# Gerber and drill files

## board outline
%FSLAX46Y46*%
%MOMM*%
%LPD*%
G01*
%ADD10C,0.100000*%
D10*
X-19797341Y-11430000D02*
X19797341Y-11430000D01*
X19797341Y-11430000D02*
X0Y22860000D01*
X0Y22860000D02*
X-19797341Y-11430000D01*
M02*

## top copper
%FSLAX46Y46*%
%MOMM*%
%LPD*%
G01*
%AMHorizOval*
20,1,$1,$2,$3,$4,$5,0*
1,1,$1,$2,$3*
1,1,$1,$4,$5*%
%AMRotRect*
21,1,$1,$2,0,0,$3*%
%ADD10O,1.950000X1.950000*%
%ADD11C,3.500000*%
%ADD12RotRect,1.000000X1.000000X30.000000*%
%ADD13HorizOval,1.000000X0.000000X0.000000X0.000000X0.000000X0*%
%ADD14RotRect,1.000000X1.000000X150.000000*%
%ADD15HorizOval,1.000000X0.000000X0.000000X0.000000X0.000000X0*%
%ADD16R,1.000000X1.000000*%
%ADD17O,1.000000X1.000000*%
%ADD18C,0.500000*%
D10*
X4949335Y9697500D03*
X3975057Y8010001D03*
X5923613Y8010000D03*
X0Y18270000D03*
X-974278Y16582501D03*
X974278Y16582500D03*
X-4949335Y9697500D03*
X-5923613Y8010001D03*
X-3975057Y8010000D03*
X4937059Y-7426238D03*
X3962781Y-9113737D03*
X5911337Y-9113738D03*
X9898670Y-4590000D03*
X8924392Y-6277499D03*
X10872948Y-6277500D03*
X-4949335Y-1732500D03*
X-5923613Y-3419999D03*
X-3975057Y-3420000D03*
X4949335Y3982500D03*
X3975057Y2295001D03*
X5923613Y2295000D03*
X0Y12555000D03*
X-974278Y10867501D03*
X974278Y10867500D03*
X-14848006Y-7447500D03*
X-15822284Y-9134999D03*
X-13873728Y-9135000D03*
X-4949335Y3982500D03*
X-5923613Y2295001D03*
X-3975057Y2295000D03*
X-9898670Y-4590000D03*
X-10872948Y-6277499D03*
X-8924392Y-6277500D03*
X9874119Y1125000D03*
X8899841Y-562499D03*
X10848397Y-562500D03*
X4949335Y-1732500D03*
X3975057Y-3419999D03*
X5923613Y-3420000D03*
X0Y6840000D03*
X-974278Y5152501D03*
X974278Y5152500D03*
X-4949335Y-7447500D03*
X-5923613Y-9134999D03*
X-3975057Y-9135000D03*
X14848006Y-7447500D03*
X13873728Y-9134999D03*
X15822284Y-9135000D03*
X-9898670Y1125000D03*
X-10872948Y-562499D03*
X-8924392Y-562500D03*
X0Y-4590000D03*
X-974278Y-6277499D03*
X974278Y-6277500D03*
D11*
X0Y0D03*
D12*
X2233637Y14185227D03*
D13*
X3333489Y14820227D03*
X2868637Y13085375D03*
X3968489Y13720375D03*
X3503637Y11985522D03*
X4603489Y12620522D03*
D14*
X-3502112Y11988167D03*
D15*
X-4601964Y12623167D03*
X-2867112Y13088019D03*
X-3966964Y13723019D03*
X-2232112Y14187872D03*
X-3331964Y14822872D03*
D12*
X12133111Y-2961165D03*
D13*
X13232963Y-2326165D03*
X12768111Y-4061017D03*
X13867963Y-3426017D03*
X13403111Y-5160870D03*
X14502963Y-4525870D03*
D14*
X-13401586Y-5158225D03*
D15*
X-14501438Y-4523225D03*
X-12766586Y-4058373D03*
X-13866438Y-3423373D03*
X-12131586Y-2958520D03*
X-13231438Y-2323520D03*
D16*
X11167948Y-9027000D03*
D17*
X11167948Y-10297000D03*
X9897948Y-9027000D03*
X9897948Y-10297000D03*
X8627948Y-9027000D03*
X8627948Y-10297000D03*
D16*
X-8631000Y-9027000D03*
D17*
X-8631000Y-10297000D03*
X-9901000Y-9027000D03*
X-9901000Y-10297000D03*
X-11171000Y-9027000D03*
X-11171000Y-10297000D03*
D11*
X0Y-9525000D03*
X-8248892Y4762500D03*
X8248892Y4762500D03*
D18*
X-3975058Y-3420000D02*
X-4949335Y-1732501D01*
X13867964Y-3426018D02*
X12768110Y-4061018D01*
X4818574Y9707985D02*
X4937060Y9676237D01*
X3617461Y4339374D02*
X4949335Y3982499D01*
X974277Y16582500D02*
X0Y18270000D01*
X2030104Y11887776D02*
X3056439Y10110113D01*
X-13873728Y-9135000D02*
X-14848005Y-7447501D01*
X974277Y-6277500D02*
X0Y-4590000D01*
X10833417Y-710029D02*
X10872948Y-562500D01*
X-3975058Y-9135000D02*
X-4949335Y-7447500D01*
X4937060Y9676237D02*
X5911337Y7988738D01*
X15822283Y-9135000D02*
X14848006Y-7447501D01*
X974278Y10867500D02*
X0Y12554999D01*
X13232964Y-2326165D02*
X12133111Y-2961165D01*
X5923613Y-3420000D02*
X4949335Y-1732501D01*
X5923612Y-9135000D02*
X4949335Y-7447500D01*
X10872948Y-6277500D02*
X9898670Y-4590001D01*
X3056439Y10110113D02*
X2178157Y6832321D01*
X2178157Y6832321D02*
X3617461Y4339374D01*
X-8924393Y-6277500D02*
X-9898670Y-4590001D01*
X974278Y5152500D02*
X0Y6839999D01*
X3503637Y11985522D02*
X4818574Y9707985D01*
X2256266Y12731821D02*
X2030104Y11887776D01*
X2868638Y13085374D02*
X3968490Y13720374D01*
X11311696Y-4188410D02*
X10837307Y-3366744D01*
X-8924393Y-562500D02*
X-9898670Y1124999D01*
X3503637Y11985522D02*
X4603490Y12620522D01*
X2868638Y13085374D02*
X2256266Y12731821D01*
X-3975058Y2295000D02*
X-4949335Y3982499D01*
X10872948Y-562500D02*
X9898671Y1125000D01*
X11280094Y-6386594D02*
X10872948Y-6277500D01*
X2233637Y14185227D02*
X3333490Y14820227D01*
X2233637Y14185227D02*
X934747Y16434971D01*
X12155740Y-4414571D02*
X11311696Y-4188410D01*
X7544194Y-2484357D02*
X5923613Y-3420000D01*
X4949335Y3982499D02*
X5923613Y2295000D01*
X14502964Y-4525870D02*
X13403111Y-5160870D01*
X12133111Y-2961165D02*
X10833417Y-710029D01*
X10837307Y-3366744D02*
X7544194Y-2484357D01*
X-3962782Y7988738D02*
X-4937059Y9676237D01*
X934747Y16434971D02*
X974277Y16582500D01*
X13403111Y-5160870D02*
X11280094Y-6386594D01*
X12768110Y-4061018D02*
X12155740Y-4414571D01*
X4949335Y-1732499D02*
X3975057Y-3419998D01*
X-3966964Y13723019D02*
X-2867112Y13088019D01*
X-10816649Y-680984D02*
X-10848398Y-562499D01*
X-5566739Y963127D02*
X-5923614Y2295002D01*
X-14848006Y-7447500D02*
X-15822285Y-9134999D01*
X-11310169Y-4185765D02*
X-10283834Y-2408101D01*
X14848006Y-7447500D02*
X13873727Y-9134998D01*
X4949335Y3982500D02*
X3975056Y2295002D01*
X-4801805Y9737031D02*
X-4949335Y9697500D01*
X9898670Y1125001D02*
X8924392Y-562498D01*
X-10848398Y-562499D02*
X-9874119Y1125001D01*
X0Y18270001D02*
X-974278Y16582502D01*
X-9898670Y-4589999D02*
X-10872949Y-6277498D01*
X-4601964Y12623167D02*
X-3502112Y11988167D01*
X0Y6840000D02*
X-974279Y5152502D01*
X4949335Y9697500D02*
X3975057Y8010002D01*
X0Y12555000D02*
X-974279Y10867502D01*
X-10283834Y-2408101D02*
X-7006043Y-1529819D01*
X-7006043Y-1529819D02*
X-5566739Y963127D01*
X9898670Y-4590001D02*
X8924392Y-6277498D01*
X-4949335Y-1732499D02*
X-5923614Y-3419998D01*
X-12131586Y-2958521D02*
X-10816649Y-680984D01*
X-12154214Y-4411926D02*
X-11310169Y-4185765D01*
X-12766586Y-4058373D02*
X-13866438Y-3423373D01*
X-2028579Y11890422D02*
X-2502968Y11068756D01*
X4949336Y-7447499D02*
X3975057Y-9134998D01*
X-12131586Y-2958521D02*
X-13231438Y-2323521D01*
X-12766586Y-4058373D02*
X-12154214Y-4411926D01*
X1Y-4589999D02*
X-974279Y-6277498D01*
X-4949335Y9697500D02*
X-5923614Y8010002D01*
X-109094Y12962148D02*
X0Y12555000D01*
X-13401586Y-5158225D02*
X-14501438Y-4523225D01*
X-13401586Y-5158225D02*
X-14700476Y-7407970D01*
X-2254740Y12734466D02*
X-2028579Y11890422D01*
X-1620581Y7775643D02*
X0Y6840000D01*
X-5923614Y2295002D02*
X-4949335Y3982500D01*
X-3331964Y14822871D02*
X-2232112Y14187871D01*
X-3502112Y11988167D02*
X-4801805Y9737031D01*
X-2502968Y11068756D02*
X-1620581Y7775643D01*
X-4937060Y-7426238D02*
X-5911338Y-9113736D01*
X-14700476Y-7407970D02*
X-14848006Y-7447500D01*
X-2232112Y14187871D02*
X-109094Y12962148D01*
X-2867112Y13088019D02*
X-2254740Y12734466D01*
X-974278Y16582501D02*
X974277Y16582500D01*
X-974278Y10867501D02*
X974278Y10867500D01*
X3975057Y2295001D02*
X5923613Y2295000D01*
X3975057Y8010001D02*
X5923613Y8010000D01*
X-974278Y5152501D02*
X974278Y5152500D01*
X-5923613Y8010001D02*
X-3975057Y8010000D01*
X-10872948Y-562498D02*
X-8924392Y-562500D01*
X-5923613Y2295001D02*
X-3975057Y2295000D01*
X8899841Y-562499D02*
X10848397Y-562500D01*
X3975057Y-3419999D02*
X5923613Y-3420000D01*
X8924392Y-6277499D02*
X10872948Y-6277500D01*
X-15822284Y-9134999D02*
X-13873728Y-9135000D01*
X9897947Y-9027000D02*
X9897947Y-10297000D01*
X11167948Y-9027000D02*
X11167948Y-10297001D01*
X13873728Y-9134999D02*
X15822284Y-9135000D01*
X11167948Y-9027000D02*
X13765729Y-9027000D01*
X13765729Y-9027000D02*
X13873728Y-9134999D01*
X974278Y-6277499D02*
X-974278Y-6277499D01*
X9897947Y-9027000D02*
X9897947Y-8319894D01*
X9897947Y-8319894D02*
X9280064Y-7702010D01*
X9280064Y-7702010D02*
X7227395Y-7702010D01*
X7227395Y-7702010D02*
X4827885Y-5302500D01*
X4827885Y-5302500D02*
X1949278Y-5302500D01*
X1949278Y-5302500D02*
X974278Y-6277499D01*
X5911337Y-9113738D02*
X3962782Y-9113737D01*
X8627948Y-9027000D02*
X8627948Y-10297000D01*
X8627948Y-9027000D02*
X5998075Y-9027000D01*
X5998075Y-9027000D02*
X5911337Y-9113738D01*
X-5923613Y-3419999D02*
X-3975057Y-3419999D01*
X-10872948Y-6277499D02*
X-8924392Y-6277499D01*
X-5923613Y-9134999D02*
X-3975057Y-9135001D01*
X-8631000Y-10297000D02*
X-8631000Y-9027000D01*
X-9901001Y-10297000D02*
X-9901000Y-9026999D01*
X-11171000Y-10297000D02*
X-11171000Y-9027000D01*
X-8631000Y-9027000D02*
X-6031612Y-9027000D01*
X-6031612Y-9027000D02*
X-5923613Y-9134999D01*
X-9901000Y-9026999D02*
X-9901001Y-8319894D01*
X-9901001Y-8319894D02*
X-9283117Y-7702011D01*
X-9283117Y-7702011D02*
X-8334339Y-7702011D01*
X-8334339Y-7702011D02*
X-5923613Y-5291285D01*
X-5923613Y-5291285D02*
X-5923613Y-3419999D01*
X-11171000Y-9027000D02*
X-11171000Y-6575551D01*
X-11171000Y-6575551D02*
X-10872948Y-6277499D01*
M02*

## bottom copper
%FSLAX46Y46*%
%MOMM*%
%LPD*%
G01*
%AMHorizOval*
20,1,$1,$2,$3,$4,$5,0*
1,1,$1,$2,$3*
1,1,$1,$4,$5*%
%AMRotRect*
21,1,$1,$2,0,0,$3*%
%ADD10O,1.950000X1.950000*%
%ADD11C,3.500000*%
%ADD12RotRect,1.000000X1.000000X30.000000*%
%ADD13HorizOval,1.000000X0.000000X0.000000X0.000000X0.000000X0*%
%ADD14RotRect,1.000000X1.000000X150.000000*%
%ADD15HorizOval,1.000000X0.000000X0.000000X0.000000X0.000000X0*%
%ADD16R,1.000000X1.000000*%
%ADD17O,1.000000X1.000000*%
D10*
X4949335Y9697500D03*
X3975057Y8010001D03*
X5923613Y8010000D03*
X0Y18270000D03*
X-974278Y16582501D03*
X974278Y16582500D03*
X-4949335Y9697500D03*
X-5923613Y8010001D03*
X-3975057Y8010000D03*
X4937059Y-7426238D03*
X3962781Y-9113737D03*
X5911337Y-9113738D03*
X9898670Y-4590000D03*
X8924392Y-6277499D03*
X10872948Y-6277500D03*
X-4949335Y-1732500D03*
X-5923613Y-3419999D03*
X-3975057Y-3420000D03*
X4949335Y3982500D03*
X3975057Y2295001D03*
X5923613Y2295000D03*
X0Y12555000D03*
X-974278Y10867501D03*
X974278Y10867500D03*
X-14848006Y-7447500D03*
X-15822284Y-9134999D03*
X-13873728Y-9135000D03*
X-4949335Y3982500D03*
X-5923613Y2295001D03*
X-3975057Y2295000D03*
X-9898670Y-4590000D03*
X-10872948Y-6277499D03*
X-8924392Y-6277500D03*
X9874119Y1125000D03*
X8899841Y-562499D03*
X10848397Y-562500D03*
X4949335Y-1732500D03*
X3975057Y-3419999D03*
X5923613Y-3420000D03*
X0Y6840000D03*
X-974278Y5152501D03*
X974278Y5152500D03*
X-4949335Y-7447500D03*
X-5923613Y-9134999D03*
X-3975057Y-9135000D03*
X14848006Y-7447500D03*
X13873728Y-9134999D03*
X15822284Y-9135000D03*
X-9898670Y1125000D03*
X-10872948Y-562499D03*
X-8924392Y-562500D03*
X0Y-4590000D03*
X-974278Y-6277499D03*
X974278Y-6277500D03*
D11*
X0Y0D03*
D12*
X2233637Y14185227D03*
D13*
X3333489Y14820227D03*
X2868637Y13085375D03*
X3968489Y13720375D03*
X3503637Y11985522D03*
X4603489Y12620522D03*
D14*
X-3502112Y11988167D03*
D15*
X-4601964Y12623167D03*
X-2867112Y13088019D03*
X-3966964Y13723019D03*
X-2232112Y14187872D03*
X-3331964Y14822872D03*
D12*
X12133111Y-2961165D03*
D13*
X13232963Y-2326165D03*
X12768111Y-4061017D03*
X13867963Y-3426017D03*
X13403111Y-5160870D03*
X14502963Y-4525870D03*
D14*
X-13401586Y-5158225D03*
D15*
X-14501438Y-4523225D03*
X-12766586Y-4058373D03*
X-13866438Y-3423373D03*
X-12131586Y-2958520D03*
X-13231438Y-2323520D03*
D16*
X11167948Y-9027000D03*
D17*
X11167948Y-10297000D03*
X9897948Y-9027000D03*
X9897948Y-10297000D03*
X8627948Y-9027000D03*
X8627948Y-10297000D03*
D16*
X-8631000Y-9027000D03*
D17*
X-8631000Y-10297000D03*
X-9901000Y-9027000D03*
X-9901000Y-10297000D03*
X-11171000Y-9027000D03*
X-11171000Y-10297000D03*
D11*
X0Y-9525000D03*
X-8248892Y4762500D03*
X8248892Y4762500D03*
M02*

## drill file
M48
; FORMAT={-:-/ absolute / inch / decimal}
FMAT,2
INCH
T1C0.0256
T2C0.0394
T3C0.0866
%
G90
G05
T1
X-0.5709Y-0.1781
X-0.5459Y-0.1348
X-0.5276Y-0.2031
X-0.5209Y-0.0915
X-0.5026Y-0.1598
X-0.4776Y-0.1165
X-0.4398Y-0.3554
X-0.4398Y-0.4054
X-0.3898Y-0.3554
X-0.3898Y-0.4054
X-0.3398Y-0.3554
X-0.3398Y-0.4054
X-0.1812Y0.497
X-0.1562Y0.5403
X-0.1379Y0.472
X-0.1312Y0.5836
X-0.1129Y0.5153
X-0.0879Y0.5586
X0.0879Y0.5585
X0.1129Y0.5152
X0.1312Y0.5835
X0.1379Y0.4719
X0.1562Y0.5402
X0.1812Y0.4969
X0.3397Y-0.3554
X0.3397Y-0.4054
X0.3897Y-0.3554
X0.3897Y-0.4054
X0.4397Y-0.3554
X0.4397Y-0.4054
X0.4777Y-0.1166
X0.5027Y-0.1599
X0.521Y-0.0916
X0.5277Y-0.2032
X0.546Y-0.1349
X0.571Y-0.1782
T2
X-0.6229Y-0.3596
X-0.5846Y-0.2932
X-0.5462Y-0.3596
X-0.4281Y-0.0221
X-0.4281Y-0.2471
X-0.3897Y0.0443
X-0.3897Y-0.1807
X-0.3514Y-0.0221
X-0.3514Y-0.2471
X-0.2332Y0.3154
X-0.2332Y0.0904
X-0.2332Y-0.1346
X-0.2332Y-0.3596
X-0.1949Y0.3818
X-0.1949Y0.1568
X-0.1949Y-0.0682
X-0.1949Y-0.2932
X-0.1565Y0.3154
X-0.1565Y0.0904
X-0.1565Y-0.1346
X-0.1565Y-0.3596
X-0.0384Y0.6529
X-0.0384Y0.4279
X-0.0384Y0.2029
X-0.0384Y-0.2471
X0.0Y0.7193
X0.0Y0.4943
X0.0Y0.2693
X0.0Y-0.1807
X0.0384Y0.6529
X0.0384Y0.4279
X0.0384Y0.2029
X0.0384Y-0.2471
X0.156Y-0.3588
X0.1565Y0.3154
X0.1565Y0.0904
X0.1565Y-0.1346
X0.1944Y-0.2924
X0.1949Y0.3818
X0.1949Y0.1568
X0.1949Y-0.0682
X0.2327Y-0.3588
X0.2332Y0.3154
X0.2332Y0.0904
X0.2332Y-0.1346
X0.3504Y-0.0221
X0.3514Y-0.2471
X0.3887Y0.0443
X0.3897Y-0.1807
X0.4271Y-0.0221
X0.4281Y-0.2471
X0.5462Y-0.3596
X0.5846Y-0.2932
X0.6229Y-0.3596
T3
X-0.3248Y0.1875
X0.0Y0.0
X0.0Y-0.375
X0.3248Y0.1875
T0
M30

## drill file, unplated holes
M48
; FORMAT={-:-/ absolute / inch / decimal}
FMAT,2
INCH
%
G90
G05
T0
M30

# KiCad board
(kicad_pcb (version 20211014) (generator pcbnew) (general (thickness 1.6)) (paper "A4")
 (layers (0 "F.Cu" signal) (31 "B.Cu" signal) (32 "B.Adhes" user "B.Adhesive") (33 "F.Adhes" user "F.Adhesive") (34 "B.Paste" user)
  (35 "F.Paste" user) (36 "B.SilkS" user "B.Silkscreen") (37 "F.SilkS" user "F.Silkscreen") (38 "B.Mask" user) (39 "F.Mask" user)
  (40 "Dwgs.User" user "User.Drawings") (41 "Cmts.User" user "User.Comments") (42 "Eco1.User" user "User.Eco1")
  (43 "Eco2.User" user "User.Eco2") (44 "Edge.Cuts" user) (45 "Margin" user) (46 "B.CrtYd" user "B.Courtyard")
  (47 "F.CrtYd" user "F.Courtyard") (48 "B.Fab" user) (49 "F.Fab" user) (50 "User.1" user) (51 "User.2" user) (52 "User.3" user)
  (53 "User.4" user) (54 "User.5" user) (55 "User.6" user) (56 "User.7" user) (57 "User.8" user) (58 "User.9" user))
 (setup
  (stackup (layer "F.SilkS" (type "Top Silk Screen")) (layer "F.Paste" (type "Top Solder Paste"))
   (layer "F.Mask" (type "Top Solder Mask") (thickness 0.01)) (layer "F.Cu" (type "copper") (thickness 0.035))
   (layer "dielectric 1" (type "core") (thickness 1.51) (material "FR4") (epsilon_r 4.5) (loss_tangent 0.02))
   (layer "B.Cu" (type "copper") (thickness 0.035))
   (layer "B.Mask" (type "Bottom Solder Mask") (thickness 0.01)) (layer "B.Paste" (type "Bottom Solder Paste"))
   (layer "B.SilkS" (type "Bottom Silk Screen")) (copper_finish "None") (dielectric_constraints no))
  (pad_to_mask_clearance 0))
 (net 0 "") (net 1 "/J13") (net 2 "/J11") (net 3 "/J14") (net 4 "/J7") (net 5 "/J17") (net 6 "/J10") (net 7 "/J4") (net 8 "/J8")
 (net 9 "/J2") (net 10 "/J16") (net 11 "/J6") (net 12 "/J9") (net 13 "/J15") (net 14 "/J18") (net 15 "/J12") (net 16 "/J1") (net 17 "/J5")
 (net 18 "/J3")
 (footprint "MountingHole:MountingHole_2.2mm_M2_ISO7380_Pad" (layer "F.Cu") (at 0 9.525)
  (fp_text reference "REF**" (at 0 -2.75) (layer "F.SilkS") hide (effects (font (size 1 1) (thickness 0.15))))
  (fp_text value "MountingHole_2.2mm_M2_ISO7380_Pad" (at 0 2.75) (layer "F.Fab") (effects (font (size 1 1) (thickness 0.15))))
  (pad "1" thru_hole circle (at 0 0) (size 3.5 3.5) (drill 2.2) (layers *.Cu *.Mask)))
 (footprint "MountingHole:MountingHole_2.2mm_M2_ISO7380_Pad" (layer "F.Cu") (at 0 0)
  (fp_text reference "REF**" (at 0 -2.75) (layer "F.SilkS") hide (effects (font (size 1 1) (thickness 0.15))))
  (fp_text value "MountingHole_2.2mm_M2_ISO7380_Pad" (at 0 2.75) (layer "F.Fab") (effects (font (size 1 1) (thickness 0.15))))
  (pad "1" thru_hole circle (at 0 0) (size 3.5 3.5) (drill 2.2) (layers *.Cu *.Mask)))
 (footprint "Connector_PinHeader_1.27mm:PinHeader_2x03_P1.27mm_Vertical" (layer "F.Cu") (at 11.167948 9.027 -90)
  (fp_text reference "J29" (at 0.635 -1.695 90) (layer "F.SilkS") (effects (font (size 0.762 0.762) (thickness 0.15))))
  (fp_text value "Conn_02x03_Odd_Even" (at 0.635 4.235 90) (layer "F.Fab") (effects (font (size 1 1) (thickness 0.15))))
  (pad "1" thru_hole rect (at 0 0 270) (size 1 1) (drill 0.65) (layers *.Cu *.Mask) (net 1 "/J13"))
  (pad "2" thru_hole oval (at 1.27 0 270) (size 1 1) (drill 0.65) (layers *.Cu *.Mask) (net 1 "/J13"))
  (pad "3" thru_hole oval (at 0 1.27 270) (size 1 1) (drill 0.65) (layers *.Cu *.Mask) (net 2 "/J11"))
  (pad "4" thru_hole oval (at 1.27 1.27 270) (size 1 1) (drill 0.65) (layers *.Cu *.Mask) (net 2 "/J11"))
  (pad "5" thru_hole oval (at 0 2.54 270) (size 1 1) (drill 0.65) (layers *.Cu *.Mask) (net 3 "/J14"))
  (pad "6" thru_hole oval (at 1.27 2.54 270) (size 1 1) (drill 0.65) (layers *.Cu *.Mask) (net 3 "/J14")))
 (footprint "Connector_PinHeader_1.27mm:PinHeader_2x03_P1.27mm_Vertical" (layer "F.Cu") (at 12.133111 2.961165 30)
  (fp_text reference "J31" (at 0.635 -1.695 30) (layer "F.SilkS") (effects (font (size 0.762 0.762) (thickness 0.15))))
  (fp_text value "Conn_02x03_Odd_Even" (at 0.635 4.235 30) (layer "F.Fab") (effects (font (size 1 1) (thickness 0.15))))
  (pad "1" thru_hole rect (at 0 0 30) (size 1 1) (drill 0.65) (layers *.Cu *.Mask) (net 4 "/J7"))
  (pad "2" thru_hole oval (at 1.27 0 30) (size 1 1) (drill 0.65) (layers *.Cu *.Mask) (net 4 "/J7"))
  (pad "3" thru_hole oval (at 0 1.27 30) (size 1 1) (drill 0.65) (layers *.Cu *.Mask) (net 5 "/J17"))
  (pad "4" thru_hole oval (at 1.27 1.27 30) (size 1 1) (drill 0.65) (layers *.Cu *.Mask) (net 5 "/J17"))
  (pad "5" thru_hole oval (at 0 2.54 30) (size 1 1) (drill 0.65) (layers *.Cu *.Mask) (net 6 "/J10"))
  (pad "6" thru_hole oval (at 1.27 2.54 30) (size 1 1) (drill 0.65) (layers *.Cu *.Mask) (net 6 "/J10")))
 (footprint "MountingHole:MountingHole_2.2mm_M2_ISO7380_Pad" (layer "F.Cu") (at -8.248892 -4.7625)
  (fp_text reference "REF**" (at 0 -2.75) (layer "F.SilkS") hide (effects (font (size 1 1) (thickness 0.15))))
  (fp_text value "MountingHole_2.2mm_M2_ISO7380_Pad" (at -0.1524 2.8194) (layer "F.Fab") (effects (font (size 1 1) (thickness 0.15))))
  (pad "1" thru_hole circle (at 0 0) (size 3.5 3.5) (drill 2.2) (layers *.Cu *.Mask)))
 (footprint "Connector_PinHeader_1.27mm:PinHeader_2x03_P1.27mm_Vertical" (layer "F.Cu") (at -3.502112 -11.988167 150)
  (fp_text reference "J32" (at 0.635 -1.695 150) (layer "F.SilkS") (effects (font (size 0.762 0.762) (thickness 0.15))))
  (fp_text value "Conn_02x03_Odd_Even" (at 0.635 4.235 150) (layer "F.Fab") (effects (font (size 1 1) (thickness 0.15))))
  (pad "1" thru_hole rect (at 0 0 150) (size 1 1) (drill 0.65) (layers *.Cu *.Mask) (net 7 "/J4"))
  (pad "2" thru_hole oval (at 1.27 0 150) (size 1 1) (drill 0.65) (layers *.Cu *.Mask) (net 7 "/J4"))
  (pad "3" thru_hole oval (at 0 1.27 150) (size 1 1) (drill 0.65) (layers *.Cu *.Mask) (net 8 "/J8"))
  (pad "4" thru_hole oval (at 1.27 1.27 150) (size 1 1) (drill 0.65) (layers *.Cu *.Mask) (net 8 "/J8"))
  (pad "5" thru_hole oval (at 0 2.54 150) (size 1 1) (drill 0.65) (layers *.Cu *.Mask) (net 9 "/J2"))
  (pad "6" thru_hole oval (at 1.27 2.54 150) (size 1 1) (drill 0.65) (layers *.Cu *.Mask) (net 9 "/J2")))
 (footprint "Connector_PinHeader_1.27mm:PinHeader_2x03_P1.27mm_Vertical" (layer "F.Cu") (at -13.401586 5.158225 150)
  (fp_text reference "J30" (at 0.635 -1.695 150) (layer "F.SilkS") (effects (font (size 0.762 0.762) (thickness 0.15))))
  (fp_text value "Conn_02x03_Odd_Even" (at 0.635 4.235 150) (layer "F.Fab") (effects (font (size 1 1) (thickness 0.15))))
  (pad "1" thru_hole rect (at 0 0 150) (size 1 1) (drill 0.65) (layers *.Cu *.Mask) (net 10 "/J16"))
  (pad "2" thru_hole oval (at 1.27 0 150) (size 1 1) (drill 0.65) (layers *.Cu *.Mask) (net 10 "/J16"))
  (pad "3" thru_hole oval (at 0 1.27 150) (size 1 1) (drill 0.65) (layers *.Cu *.Mask) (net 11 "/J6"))
  (pad "4" thru_hole oval (at 1.27 1.27 150) (size 1 1) (drill 0.65) (layers *.Cu *.Mask) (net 11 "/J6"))
  (pad "5" thru_hole oval (at 0 2.54 150) (size 1 1) (drill 0.65) (layers *.Cu *.Mask) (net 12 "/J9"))
  (pad "6" thru_hole oval (at 1.27 2.54 150) (size 1 1) (drill 0.65) (layers *.Cu *.Mask) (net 12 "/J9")))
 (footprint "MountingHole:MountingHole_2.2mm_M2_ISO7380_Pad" (layer "F.Cu") (at 8.248892 -4.7625)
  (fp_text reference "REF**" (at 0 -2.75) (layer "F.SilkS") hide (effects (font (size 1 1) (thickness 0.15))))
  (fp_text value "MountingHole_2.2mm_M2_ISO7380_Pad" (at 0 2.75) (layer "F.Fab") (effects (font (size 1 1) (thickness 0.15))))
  (pad "1" thru_hole circle (at 0 0) (size 3.5 3.5) (drill 2.2) (layers *.Cu *.Mask)))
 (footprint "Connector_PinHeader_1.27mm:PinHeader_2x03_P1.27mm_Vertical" (layer "F.Cu") (at -8.631 9.027 -90)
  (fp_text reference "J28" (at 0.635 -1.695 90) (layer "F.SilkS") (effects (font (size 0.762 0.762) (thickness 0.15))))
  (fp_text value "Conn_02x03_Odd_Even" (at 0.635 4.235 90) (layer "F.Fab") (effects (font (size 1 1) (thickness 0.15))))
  (pad "1" thru_hole rect (at 0 0 270) (size 1 1) (drill 0.65) (layers *.Cu *.Mask) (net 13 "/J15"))
  (pad "2" thru_hole oval (at 1.27 0 270) (size 1 1) (drill 0.65) (layers *.Cu *.Mask) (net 13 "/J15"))
  (pad "3" thru_hole oval (at 0 1.27 270) (size 1 1) (drill 0.65) (layers *.Cu *.Mask) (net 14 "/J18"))
  (pad "4" thru_hole oval (at 1.27 1.27 270) (size 1 1) (drill 0.65) (layers *.Cu *.Mask) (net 14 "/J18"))
  (pad "5" thru_hole oval (at 0 2.54 270) (size 1 1) (drill 0.65) (layers *.Cu *.Mask) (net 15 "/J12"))
  (pad "6" thru_hole oval (at 1.27 2.54 270) (size 1 1) (drill 0.65) (layers *.Cu *.Mask) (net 15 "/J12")))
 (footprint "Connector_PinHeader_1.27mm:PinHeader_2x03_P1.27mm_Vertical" (layer "F.Cu") (at 2.233637 -14.185227 30)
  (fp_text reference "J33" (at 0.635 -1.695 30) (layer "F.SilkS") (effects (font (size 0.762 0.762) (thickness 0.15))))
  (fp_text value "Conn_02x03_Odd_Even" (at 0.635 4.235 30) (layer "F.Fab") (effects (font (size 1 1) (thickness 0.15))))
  (pad "1" thru_hole rect (at 0 0 30) (size 1 1) (drill 0.65) (layers *.Cu *.Mask) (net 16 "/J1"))
  (pad "2" thru_hole oval (at 1.27 0 30) (size 1 1) (drill 0.65) (layers *.Cu *.Mask) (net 16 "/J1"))
  (pad "3" thru_hole oval (at 0 1.27 30) (size 1 1) (drill 0.65) (layers *.Cu *.Mask) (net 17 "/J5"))
  (pad "4" thru_hole oval (at 1.27 1.27 30) (size 1 1) (drill 0.65) (layers *.Cu *.Mask) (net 17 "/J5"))
  (pad "5" thru_hole oval (at 0 2.54 30) (size 1 1) (drill 0.65) (layers *.Cu *.Mask) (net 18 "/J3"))
  (pad "6" thru_hole oval (at 1.27 2.54 30) (size 1 1) (drill 0.65) (layers *.Cu *.Mask) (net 18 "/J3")))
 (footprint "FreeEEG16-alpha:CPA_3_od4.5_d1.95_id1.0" (layer "B.Cu") (at 0 -17.145 180)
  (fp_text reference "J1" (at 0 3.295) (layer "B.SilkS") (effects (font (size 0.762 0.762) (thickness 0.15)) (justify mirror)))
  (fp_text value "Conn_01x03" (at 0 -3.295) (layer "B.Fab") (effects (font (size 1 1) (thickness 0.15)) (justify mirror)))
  (pad "1" thru_hole oval (at 0 1.125 180) (size 1.95 1.95) (drill 1) (layers *.Cu *.Mask) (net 16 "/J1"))
  (pad "2" thru_hole oval (at 0.974278 -0.562499 180) (size 1.95 1.95) (drill 1) (layers *.Cu *.Mask) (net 16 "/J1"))
  (pad "3" thru_hole oval (at -0.974278 -0.5625 180) (size 1.95 1.95) (drill 1) (layers *.Cu *.Mask) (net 16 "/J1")))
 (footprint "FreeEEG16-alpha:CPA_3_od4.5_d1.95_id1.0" (layer "B.Cu") (at -4.949335 -8.5725 180)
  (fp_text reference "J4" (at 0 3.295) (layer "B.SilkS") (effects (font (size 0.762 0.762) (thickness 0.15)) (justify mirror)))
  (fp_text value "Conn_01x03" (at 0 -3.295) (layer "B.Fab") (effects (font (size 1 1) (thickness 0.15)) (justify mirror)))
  (pad "1" thru_hole oval (at 0 1.125 180) (size 1.95 1.95) (drill 1) (layers *.Cu *.Mask) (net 7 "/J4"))
  (pad "2" thru_hole oval (at 0.974278 -0.562499 180) (size 1.95 1.95) (drill 1) (layers *.Cu *.Mask) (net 7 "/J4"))
  (pad "3" thru_hole oval (at -0.974278 -0.5625 180) (size 1.95 1.95) (drill 1) (layers *.Cu *.Mask) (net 7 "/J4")))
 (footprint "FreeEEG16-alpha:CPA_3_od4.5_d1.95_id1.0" (layer "B.Cu") (at 4.937059 8.551238 180)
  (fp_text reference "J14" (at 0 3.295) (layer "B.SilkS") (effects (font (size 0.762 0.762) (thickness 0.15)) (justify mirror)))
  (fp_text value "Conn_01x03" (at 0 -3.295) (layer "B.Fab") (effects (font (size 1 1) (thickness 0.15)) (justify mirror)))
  (pad "1" thru_hole oval (at 0 1.125 180) (size 1.95 1.95) (drill 1) (layers *.Cu *.Mask) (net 3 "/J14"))
  (pad "2" thru_hole oval (at 0.974278 -0.562499 180) (size 1.95 1.95) (drill 1) (layers *.Cu *.Mask) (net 3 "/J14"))
  (pad "3" thru_hole oval (at -0.974278 -0.5625 180) (size 1.95 1.95) (drill 1) (layers *.Cu *.Mask) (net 3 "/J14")))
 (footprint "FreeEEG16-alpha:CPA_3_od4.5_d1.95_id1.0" (layer "B.Cu") (at 4.949335 -8.5725 180)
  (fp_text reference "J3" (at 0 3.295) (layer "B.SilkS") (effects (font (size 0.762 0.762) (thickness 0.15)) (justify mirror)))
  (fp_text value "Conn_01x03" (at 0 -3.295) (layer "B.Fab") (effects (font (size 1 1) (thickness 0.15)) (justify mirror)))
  (pad "1" thru_hole oval (at 0 1.125 180) (size 1.95 1.95) (drill 1) (layers *.Cu *.Mask) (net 18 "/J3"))
  (pad "2" thru_hole oval (at 0.974278 -0.562499 180) (size 1.95 1.95) (drill 1) (layers *.Cu *.Mask) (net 18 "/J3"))
  (pad "3" thru_hole oval (at -0.974278 -0.5625 180) (size 1.95 1.95) (drill 1) (layers *.Cu *.Mask) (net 18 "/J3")))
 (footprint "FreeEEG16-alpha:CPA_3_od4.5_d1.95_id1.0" (layer "B.Cu") (at 9.89867 5.715 180)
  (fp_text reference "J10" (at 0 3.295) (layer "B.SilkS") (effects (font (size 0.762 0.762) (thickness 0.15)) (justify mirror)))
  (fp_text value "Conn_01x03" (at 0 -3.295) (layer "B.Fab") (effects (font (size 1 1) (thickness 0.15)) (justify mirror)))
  (pad "1" thru_hole oval (at 0 1.125 180) (size 1.95 1.95) (drill 1) (layers *.Cu *.Mask) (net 6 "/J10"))
  (pad "2" thru_hole oval (at 0.974278 -0.562499 180) (size 1.95 1.95) (drill 1) (layers *.Cu *.Mask) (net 6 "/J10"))
  (pad "3" thru_hole oval (at -0.974278 -0.5625 180) (size 1.95 1.95) (drill 1) (layers *.Cu *.Mask) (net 6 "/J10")))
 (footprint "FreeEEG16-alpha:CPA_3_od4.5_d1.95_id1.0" (layer "B.Cu") (at -4.949335 2.8575 180)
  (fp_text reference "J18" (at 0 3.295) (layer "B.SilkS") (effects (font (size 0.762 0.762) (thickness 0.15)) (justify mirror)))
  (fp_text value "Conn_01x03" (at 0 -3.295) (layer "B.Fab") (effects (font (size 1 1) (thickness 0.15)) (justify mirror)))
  (pad "1" thru_hole oval (at 0 1.125 180) (size 1.95 1.95) (drill 1) (layers *.Cu *.Mask) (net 14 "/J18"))
  (pad "2" thru_hole oval (at 0.974278 -0.562499 180) (size 1.95 1.95) (drill 1) (layers *.Cu *.Mask) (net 14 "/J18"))
  (pad "3" thru_hole oval (at -0.974278 -0.5625 180) (size 1.95 1.95) (drill 1) (layers *.Cu *.Mask) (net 14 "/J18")))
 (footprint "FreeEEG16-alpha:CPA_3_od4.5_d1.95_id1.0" (layer "B.Cu") (at 4.949335 -2.8575 180)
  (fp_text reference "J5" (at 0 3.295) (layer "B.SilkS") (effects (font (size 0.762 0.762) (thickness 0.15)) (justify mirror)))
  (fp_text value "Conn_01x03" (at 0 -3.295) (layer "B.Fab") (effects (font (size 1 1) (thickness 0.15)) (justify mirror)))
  (pad "1" thru_hole oval (at 0 1.125 180) (size 1.95 1.95) (drill 1) (layers *.Cu *.Mask) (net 17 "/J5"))
  (pad "2" thru_hole oval (at 0.974278 -0.562499 180) (size 1.95 1.95) (drill 1) (layers *.Cu *.Mask) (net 17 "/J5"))
  (pad "3" thru_hole oval (at -0.974278 -0.5625 180) (size 1.95 1.95) (drill 1) (layers *.Cu *.Mask) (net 17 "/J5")))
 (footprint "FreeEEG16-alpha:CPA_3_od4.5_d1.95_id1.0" (layer "B.Cu") (at 0 -11.43 180)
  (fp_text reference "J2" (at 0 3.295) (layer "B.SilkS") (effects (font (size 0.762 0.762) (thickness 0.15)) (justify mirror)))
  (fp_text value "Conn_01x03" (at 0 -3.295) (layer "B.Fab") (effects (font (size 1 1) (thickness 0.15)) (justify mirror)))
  (pad "1" thru_hole oval (at 0 1.125 180) (size 1.95 1.95) (drill 1) (layers *.Cu *.Mask) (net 9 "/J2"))
  (pad "2" thru_hole oval (at 0.974278 -0.562499 180) (size 1.95 1.95) (drill 1) (layers *.Cu *.Mask) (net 9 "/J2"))
  (pad "3" thru_hole oval (at -0.974278 -0.5625 180) (size 1.95 1.95) (drill 1) (layers *.Cu *.Mask) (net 9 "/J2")))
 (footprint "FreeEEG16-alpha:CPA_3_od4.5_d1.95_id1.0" (layer "B.Cu") (at -14.848006 8.5725 180)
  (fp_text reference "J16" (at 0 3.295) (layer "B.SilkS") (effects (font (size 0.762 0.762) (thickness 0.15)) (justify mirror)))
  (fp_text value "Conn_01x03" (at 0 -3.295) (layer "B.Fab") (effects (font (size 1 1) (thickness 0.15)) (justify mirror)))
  (pad "1" thru_hole oval (at 0 1.125 180) (size 1.95 1.95) (drill 1) (layers *.Cu *.Mask) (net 10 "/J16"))
  (pad "2" thru_hole oval (at 0.974278 -0.562499 180) (size 1.95 1.95) (drill 1) (layers *.Cu *.Mask) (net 10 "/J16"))
  (pad "3" thru_hole oval (at -0.974278 -0.5625 180) (size 1.95 1.95) (drill 1) (layers *.Cu *.Mask) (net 10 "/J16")))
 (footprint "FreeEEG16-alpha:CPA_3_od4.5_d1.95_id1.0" (layer "B.Cu") (at -4.949335 -2.8575 180)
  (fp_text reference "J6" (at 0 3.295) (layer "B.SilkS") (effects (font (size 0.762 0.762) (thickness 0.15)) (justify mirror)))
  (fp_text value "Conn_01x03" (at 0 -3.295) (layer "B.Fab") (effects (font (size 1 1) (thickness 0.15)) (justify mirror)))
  (pad "1" thru_hole oval (at 0 1.125 180) (size 1.95 1.95) (drill 1) (layers *.Cu *.Mask) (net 11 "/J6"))
  (pad "2" thru_hole oval (at 0.974278 -0.562499 180) (size 1.95 1.95) (drill 1) (layers *.Cu *.Mask) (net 11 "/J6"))
  (pad "3" thru_hole oval (at -0.974278 -0.5625 180) (size 1.95 1.95) (drill 1) (layers *.Cu *.Mask) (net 11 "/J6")))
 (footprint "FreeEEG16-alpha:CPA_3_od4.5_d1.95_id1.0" (layer "B.Cu") (at -9.89867 5.715 180)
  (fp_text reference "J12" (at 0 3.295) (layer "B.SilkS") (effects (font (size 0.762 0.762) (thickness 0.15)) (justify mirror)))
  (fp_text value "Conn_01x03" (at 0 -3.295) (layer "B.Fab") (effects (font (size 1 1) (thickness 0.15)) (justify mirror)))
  (pad "1" thru_hole oval (at 0 1.125 180) (size 1.95 1.95) (drill 1) (layers *.Cu *.Mask) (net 15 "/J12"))
  (pad "2" thru_hole oval (at 0.974278 -0.562499 180) (size 1.95 1.95) (drill 1) (layers *.Cu *.Mask) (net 15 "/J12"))
  (pad "3" thru_hole oval (at -0.974278 -0.5625 180) (size 1.95 1.95) (drill 1) (layers *.Cu *.Mask) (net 15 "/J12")))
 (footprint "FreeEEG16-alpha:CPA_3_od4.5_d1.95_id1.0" (layer "B.Cu") (at 9.874119 0 180)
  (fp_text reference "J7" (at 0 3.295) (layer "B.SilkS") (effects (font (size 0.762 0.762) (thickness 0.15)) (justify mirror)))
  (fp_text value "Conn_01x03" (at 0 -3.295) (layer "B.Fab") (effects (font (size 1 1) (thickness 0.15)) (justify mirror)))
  (pad "1" thru_hole oval (at 0 1.125 180) (size 1.95 1.95) (drill 1) (layers *.Cu *.Mask) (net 4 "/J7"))
  (pad "2" thru_hole oval (at 0.974278 -0.562499 180) (size 1.95 1.95) (drill 1) (layers *.Cu *.Mask) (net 4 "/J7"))
  (pad "3" thru_hole oval (at -0.974278 -0.5625 180) (size 1.95 1.95) (drill 1) (layers *.Cu *.Mask) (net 4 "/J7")))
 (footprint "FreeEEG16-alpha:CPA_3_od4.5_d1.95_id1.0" (layer "B.Cu") (at 4.949335 2.8575 180)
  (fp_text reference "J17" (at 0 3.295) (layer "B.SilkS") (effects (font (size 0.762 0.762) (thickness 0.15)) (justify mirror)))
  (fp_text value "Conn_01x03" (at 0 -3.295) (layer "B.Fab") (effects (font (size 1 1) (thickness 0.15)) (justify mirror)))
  (pad "1" thru_hole oval (at 0 1.125 180) (size 1.95 1.95) (drill 1) (layers *.Cu *.Mask) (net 5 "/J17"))
  (pad "2" thru_hole oval (at 0.974278 -0.562499 180) (size 1.95 1.95) (drill 1) (layers *.Cu *.Mask) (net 5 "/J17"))
  (pad "3" thru_hole oval (at -0.974278 -0.5625 180) (size 1.95 1.95) (drill 1) (layers *.Cu *.Mask) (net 5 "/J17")))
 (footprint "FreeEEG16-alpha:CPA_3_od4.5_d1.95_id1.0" (layer "B.Cu") (at 0 -5.715 180)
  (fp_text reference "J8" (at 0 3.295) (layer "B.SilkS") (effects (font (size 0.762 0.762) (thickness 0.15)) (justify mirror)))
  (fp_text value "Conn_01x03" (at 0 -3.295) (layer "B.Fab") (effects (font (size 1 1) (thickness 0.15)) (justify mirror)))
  (pad "1" thru_hole oval (at 0 1.125 180) (size 1.95 1.95) (drill 1) (layers *.Cu *.Mask) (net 8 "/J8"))
  (pad "2" thru_hole oval (at 0.974278 -0.562499 180) (size 1.95 1.95) (drill 1) (layers *.Cu *.Mask) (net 8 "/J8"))
  (pad "3" thru_hole oval (at -0.974278 -0.5625 180) (size 1.95 1.95) (drill 1) (layers *.Cu *.Mask) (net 8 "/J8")))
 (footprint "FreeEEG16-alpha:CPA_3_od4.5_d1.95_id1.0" (layer "B.Cu") (at -4.949335 8.5725 180)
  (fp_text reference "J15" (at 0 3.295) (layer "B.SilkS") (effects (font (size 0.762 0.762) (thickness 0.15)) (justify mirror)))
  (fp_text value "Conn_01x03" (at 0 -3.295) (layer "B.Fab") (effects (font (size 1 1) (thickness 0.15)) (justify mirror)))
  (pad "1" thru_hole oval (at 0 1.125 180) (size 1.95 1.95) (drill 1) (layers *.Cu *.Mask) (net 13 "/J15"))
  (pad "2" thru_hole oval (at 0.974278 -0.562499 180) (size 1.95 1.95) (drill 1) (layers *.Cu *.Mask) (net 13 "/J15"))
  (pad "3" thru_hole oval (at -0.974278 -0.5625 180) (size 1.95 1.95) (drill 1) (layers *.Cu *.Mask) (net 13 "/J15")))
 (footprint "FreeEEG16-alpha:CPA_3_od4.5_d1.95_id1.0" (layer "B.Cu") (at 14.848006 8.5725 180)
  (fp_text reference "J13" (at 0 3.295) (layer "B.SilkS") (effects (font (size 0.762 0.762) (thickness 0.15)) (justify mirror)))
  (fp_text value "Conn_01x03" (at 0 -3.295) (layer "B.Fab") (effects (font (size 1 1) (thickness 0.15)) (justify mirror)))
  (pad "1" thru_hole oval (at 0 1.125 180) (size 1.95 1.95) (drill 1) (layers *.Cu *.Mask) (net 1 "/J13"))
  (pad "2" thru_hole oval (at 0.974278 -0.562499 180) (size 1.95 1.95) (drill 1) (layers *.Cu *.Mask) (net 1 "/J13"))
  (pad "3" thru_hole oval (at -0.974278 -0.5625 180) (size 1.95 1.95) (drill 1) (layers *.Cu *.Mask) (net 1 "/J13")))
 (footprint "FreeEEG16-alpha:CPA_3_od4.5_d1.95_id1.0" (layer "B.Cu") (at -9.89867 0 180)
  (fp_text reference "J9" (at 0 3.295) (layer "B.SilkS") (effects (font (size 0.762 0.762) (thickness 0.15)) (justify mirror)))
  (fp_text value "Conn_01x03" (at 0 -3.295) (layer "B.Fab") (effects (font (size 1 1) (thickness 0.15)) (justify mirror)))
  (pad "1" thru_hole oval (at 0 1.125 180) (size 1.95 1.95) (drill 1) (layers *.Cu *.Mask) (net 12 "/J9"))
  (pad "2" thru_hole oval (at 0.974278 -0.562499 180) (size 1.95 1.95) (drill 1) (layers *.Cu *.Mask) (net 12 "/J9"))
  (pad "3" thru_hole oval (at -0.974278 -0.5625 180) (size 1.95 1.95) (drill 1) (layers *.Cu *.Mask) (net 12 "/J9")))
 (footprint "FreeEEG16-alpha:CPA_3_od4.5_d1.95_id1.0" (layer "B.Cu") (at 0 5.715 180)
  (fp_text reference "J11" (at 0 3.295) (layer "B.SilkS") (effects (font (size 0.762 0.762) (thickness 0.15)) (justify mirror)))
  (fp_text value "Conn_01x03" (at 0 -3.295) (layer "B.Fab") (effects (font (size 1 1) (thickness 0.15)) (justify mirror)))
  (pad "1" thru_hole oval (at 0 1.125 180) (size 1.95 1.95) (drill 1) (layers *.Cu *.Mask) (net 2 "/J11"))
  (pad "2" thru_hole oval (at 0.974278 -0.562499 180) (size 1.95 1.95) (drill 1) (layers *.Cu *.Mask) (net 2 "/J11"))
  (pad "3" thru_hole oval (at -0.974278 -0.5625 180) (size 1.95 1.95) (drill 1) (layers *.Cu *.Mask) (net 2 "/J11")))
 (gr_line (start -19.797341 11.43) (end 19.797341 11.43) (layer "Edge.Cuts") (width 0.1))
 (gr_line (start 19.797341 11.43) (end 0 -22.86) (layer "Edge.Cuts") (width 0.1))
 (gr_line (start 0 -22.86) (end -19.797341 11.43) (layer "Edge.Cuts") (width 0.1))
 (segment (start 0 -18.270001) (end -0.974278 -16.582502) (width 0.5) (layer "F.Cu") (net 16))
 (segment (start 0.934747 -16.434971) (end 0.974277 -16.5825) (width 0.5) (layer "F.Cu") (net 16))
 (segment (start 0.974277 -16.5825) (end 0 -18.27) (width 0.5) (layer "F.Cu") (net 16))
 (segment (start -0.974278 -16.582501) (end 0.974277 -16.5825) (width 0.5) (layer "F.Cu") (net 16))
 (segment (start 2.233637 -14.185227) (end 0.934747 -16.434971) (width 0.5) (layer "F.Cu") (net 16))
 (segment (start 2.233637 -14.185227) (end 3.33349 -14.820227) (width 0.5) (layer "F.Cu") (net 16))
 (segment (start -2.232112 -14.187871) (end -0.109094 -12.962148) (width 0.5) (layer "F.Cu") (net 9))
 (segment (start 0 -12.555) (end -0.974279 -10.867502) (width 0.5) (layer "F.Cu") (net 9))
 (segment (start -0.974278 -10.867501) (end 0.974278 -10.8675) (width 0.5) (layer "F.Cu") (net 9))
 (segment (start -3.331964 -14.822871) (end -2.232112 -14.187871) (width 0.5) (layer "F.Cu") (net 9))
 (segment (start -0.109094 -12.962148) (end 0 -12.555) (width 0.5) (layer "F.Cu") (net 9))
 (segment (start 0.974278 -10.8675) (end 0 -12.554999) (width 0.5) (layer "F.Cu") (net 9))
 (segment (start 4.818574 -9.707985) (end 4.93706 -9.676237) (width 0.5) (layer "F.Cu") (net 18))
 (segment (start 3.503637 -11.985522) (end 4.818574 -9.707985) (width 0.5) (layer "F.Cu") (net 18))
 (segment (start 3.975057 -8.010001) (end 5.923613 -8.01) (width 0.5) (layer "F.Cu") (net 18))
 (segment (start 4.93706 -9.676237) (end 5.911337 -7.988738) (width 0.5) (layer "F.Cu") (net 18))
 (segment (start 4.949335 -9.6975) (end 3.975057 -8.010002) (width 0.5) (layer "F.Cu") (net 18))
 (segment (start 3.503637 -11.985522) (end 4.60349 -12.620522) (width 0.5) (layer "F.Cu") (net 18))
 (segment (start -4.601964 -12.623167) (end -3.502112 -11.988167) (width 0.5) (layer "F.Cu") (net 7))
 (segment (start -3.962782 -7.988738) (end -4.937059 -9.676237) (width 0.5) (layer "F.Cu") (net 7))
 (segment (start -4.801805 -9.737031) (end -4.949335 -9.6975) (width 0.5) (layer "F.Cu") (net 7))
 (segment (start -3.502112 -11.988167) (end -4.801805 -9.737031) (width 0.5) (layer "F.Cu") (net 7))
 (segment (start -5.923613 -8.010001) (end -3.975057 -8.01) (width 0.5) (layer "F.Cu") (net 7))
 (segment (start -4.949335 -9.6975) (end -5.923614 -8.010002) (width 0.5) (layer "F.Cu") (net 7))
 (segment (start 4.949335 -3.9825) (end 3.975056 -2.295002) (width 0.5) (layer "F.Cu") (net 17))
 (segment (start 2.178157 -6.832321) (end 3.617461 -4.339374) (width 0.5) (layer "F.Cu") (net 17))
 (segment (start 4.949335 -3.982499) (end 5.923613 -2.295) (width 0.5) (layer "F.Cu") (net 17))
 (segment (start 3.975057 -2.295001) (end 5.923613 -2.295) (width 0.5) (layer "F.Cu") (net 17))
 (segment (start 3.056439 -10.110113) (end 2.178157 -6.832321) (width 0.5) (layer "F.Cu") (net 17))
 (segment (start 2.030104 -11.887776) (end 3.056439 -10.110113) (width 0.5) (layer "F.Cu") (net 17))
 (segment (start 2.868638 -13.085374) (end 3.96849 -13.720374) (width 0.5) (layer "F.Cu") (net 17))
 (segment (start 2.868638 -13.085374) (end 2.256266 -12.731821) (width 0.5) (layer "F.Cu") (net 17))
 (segment (start 3.617461 -4.339374) (end 4.949335 -3.982499) (width 0.5) (layer "F.Cu") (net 17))
 (segment (start 2.256266 -12.731821) (end 2.030104 -11.887776) (width 0.5) (layer "F.Cu") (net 17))
 (segment (start -3.975058 -2.295) (end -4.949335 -3.982499) (width 0.5) (layer "F.Cu") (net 11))
 (segment (start -7.006043 1.529819) (end -5.566739 -0.963127) (width 0.5) (layer "F.Cu") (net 11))
 (segment (start -11.310169 4.185765) (end -10.283834 2.408101) (width 0.5) (layer "F.Cu") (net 11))
 (segment (start -5.923613 -2.295001) (end -3.975057 -2.295) (width 0.5) (layer "F.Cu") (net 11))
 (segment (start -10.283834 2.408101) (end -7.006043 1.529819) (width 0.5) (layer "F.Cu") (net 11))
 (segment (start -12.154214 4.411926) (end -11.310169 4.185765) (width 0.5) (layer "F.Cu") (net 11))
 (segment (start -12.766586 4.058373) (end -13.866438 3.423373) (width 0.5) (layer "F.Cu") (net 11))
 (segment (start -5.923614 -2.295002) (end -4.949335 -3.9825) (width 0.5) (layer "F.Cu") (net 11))
 (segment (start -5.566739 -0.963127) (end -5.923614 -2.295002) (width 0.5) (layer "F.Cu") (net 11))
 (segment (start -12.766586 4.058373) (end -12.154214 4.411926) (width 0.5) (layer "F.Cu") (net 11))
 (segment (start -2.028579 -11.890422) (end -2.502968 -11.068756) (width 0.5) (layer "F.Cu") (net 8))
 (segment (start -2.25474 -12.734466) (end -2.028579 -11.890422) (width 0.5) (layer "F.Cu") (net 8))
 (segment (start 0.974278 -5.1525) (end 0 -6.839999) (width 0.5) (layer "F.Cu") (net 8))
 (segment (start -1.620581 -7.775643) (end 0 -6.84) (width 0.5) (layer "F.Cu") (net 8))
 (segment (start -3.966964 -13.723019) (end -2.867112 -13.088019) (width 0.5) (layer "F.Cu") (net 8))
 (segment (start 0 -6.84) (end -0.974279 -5.152502) (width 0.5) (layer "F.Cu") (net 8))
 (segment (start -2.502968 -11.068756) (end -1.620581 -7.775643) (width 0.5) (layer "F.Cu") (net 8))
 (segment (start -0.974278 -5.152501) (end 0.974278 -5.1525) (width 0.5) (layer "F.Cu") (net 8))
 (segment (start -2.867112 -13.088019) (end -2.25474 -12.734466) (width 0.5) (layer "F.Cu") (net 8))
 (segment (start 14.502964 4.52587) (end 13.403111 5.16087) (width 0.5) (layer "F.Cu") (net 6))
 (segment (start 13.403111 5.16087) (end 11.280094 6.386594) (width 0.5) (layer "F.Cu") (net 6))
 (segment (start 9.89867 4.590001) (end 8.924392 6.277498) (width 0.5) (layer "F.Cu") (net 6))
 (segment (start 10.872948 6.2775) (end 9.89867 4.590001) (width 0.5) (layer "F.Cu") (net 6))
 (segment (start 11.280094 6.386594) (end 10.872948 6.2775) (width 0.5) (layer "F.Cu") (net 6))
 (segment (start 8.924392 6.277499) (end 10.872948 6.2775) (width 0.5) (layer "F.Cu") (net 6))
 (segment (start 9.280064 7.70201) (end 7.227395 7.70201) (width 0.5) (layer "F.Cu") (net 2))
 (segment (start 0.974277 6.2775) (end 0 4.59) (width 0.5) (layer "F.Cu") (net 2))
 (segment (start 0.974278 6.277499) (end -0.974278 6.277499) (width 0.5) (layer "F.Cu") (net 2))
 (segment (start 7.227395 7.70201) (end 4.827885 5.3025) (width 0.5) (layer "F.Cu") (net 2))
 (segment (start 0.000001 4.589999) (end -0.974279 6.277498) (width 0.5) (layer "F.Cu") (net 2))
 (segment (start 4.827885 5.3025) (end 1.949278 5.3025) (width 0.5) (layer "F.Cu") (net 2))
 (segment (start 1.949278 5.3025) (end 0.974278 6.277499) (width 0.5) (layer "F.Cu") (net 2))
 (segment (start 9.897947 8.319894) (end 9.280064 7.70201) (width 0.5) (layer "F.Cu") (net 2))
 (segment (start 9.897947 9.027) (end 9.897947 10.297) (width 0.5) (layer "F.Cu") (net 2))
 (segment (start 9.897947 9.027) (end 9.897947 8.319894) (width 0.5) (layer "F.Cu") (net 2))
 (segment (start -11.171 9.027) (end -11.171 6.575551) (width 0.5) (layer "F.Cu") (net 15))
 (segment (start -8.924393 6.2775) (end -9.89867 4.590001) (width 0.5) (layer "F.Cu") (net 15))
 (segment (start -11.171 6.575551) (end -10.872948 6.277499) (width 0.5) (layer "F.Cu") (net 15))
 (segment (start -11.171 10.297) (end -11.171 9.027) (width 0.5) (layer "F.Cu") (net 15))
 (segment (start -10.872948 6.277499) (end -8.924392 6.277499) (width 0.5) (layer "F.Cu") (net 15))
 (segment (start -9.89867 4.589999) (end -10.872949 6.277498) (width 0.5) (layer "F.Cu") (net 15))
 (segment (start 11.167948 9.027) (end 11.167948 10.297001) (width 0.5) (layer "F.Cu") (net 1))
 (segment (start 13.765729 9.027) (end 13.873728 9.134999) (width 0.5) (layer "F.Cu") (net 1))
 (segment (start 14.848006 7.4475) (end 13.873727 9.134998) (width 0.5) (layer "F.Cu") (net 1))
 (segment (start 15.822283 9.135) (end 14.848006 7.447501) (width 0.5) (layer "F.Cu") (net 1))
 (segment (start 11.167948 9.027) (end 13.765729 9.027) (width 0.5) (layer "F.Cu") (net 1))
 (segment (start 13.873728 9.134999) (end 15.822284 9.135) (width 0.5) (layer "F.Cu") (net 1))
 (segment (start 5.923612 9.135) (end 4.949335 7.4475) (width 0.5) (layer "F.Cu") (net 3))
 (segment (start 8.627948 9.027) (end 8.627948 10.297) (width 0.5) (layer "F.Cu") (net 3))
 (segment (start 5.911337 9.113738) (end 3.962782 9.113737) (width 0.5) (layer "F.Cu") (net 3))
 (segment (start 4.949336 7.447499) (end 3.975057 9.134998) (width 0.5) (layer "F.Cu") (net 3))
 (segment (start 8.627948 9.027) (end 5.998075 9.027) (width 0.5) (layer "F.Cu") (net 3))
 (segment (start 5.998075 9.027) (end 5.911337 9.113738) (width 0.5) (layer "F.Cu") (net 3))
 (segment (start -8.631 10.297) (end -8.631 9.027) (width 0.5) (layer "F.Cu") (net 13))
 (segment (start -3.975058 9.135) (end -4.949335 7.4475) (width 0.5) (layer "F.Cu") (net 13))
 (segment (start -5.923613 9.134999) (end -3.975057 9.135001) (width 0.5) (layer "F.Cu") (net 13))
 (segment (start -6.031612 9.027) (end -5.923613 9.134999) (width 0.5) (layer "F.Cu") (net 13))
 (segment (start -8.631 9.027) (end -6.031612 9.027) (width 0.5) (layer "F.Cu") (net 13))
 (segment (start -4.93706 7.426238) (end -5.911338 9.113736) (width 0.5) (layer "F.Cu") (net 13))
 (segment (start -15.822284 9.134999) (end -13.873728 9.135) (width 0.5) (layer "F.Cu") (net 10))
 (segment (start -14.848006 7.4475) (end -15.822285 9.134999) (width 0.5) (layer "F.Cu") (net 10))
 (segment (start -13.401586 5.158225) (end -14.501438 4.523225) (width 0.5) (layer "F.Cu") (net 10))
 (segment (start -14.700476 7.40797) (end -14.848006 7.4475) (width 0.5) (layer "F.Cu") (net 10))
 (segment (start -13.401586 5.158225) (end -14.700476 7.40797) (width 0.5) (layer "F.Cu") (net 10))
 (segment (start -13.873728 9.135) (end -14.848005 7.447501) (width 0.5) (layer "F.Cu") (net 10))
 (segment (start 12.76811 4.061018) (end 12.15574 4.414571) (width 0.5) (layer "F.Cu") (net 5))
 (segment (start 11.311696 4.18841) (end 10.837307 3.366744) (width 0.5) (layer "F.Cu") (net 5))
 (segment (start 3.975057 3.419999) (end 5.923613 3.42) (width 0.5) (layer "F.Cu") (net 5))
 (segment (start 4.949335 1.732499) (end 3.975057 3.419998) (width 0.5) (layer "F.Cu") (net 5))
 (segment (start 10.837307 3.366744) (end 7.544194 2.484357) (width 0.5) (layer "F.Cu") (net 5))
 (segment (start 12.15574 4.414571) (end 11.311696 4.18841) (width 0.5) (layer "F.Cu") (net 5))
 (segment (start 5.923613 3.42) (end 4.949335 1.732501) (width 0.5) (layer "F.Cu") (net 5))
 (segment (start 7.544194 2.484357) (end 5.923613 3.42) (width 0.5) (layer "F.Cu") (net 5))
 (segment (start 13.867964 3.426018) (end 12.76811 4.061018) (width 0.5) (layer "F.Cu") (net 5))
 (segment (start -9.901001 10.297) (end -9.901 9.026999) (width 0.5) (layer "F.Cu") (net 14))
 (segment (start -5.923613 3.419999) (end -3.975057 3.419999) (width 0.5) (layer "F.Cu") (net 14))
 (segment (start -4.949335 1.732499) (end -5.923614 3.419998) (width 0.5) (layer "F.Cu") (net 14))
 (segment (start -8.334339 7.702011) (end -5.923613 5.291285) (width 0.5) (layer "F.Cu") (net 14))
 (segment (start -9.901 9.026999) (end -9.901001 8.319894) (width 0.5) (layer "F.Cu") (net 14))
 (segment (start -9.901001 8.319894) (end -9.283117 7.702011) (width 0.5) (layer "F.Cu") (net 14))
 (segment (start -9.283117 7.702011) (end -8.334339 7.702011) (width 0.5) (layer "F.Cu") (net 14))
 (segment (start -5.923613 5.291285) (end -5.923613 3.419999) (width 0.5) (layer "F.Cu") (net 14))
 (segment (start -3.975058 3.42) (end -4.949335 1.732501) (width 0.5) (layer "F.Cu") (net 14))
 (segment (start -8.924393 0.5625) (end -9.89867 -1.124999) (width 0.5) (layer "F.Cu") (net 12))
 (segment (start -10.872948 0.562498) (end -8.924392 0.5625) (width 0.5) (layer "F.Cu") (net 12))
 (segment (start -12.131586 2.958521) (end -10.816649 0.680984) (width 0.5) (layer "F.Cu") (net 12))
 (segment (start -10.848398 0.562499) (end -9.874119 -1.125001) (width 0.5) (layer "F.Cu") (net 12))
 (segment (start -10.816649 0.680984) (end -10.848398 0.562499) (width 0.5) (layer "F.Cu") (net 12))
 (segment (start -12.131586 2.958521) (end -13.231438 2.323521) (width 0.5) (layer "F.Cu") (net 12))
 (segment (start 10.872948 0.5625) (end 9.898671 -1.125) (width 0.5) (layer "F.Cu") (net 4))
 (segment (start 13.232964 2.326165) (end 12.133111 2.961165) (width 0.5) (layer "F.Cu") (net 4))
 (segment (start 10.833417 0.710029) (end 10.872948 0.5625) (width 0.5) (layer "F.Cu") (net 4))
 (segment (start 9.89867 -1.125001) (end 8.924392 0.562498) (width 0.5) (layer "F.Cu") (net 4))
 (segment (start 8.899841 0.562499) (end 10.848397 0.5625) (width 0.5) (layer "F.Cu") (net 4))
 (segment (start 12.133111 2.961165) (end 10.833417 0.710029) (width 0.5) (layer "F.Cu") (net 4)))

